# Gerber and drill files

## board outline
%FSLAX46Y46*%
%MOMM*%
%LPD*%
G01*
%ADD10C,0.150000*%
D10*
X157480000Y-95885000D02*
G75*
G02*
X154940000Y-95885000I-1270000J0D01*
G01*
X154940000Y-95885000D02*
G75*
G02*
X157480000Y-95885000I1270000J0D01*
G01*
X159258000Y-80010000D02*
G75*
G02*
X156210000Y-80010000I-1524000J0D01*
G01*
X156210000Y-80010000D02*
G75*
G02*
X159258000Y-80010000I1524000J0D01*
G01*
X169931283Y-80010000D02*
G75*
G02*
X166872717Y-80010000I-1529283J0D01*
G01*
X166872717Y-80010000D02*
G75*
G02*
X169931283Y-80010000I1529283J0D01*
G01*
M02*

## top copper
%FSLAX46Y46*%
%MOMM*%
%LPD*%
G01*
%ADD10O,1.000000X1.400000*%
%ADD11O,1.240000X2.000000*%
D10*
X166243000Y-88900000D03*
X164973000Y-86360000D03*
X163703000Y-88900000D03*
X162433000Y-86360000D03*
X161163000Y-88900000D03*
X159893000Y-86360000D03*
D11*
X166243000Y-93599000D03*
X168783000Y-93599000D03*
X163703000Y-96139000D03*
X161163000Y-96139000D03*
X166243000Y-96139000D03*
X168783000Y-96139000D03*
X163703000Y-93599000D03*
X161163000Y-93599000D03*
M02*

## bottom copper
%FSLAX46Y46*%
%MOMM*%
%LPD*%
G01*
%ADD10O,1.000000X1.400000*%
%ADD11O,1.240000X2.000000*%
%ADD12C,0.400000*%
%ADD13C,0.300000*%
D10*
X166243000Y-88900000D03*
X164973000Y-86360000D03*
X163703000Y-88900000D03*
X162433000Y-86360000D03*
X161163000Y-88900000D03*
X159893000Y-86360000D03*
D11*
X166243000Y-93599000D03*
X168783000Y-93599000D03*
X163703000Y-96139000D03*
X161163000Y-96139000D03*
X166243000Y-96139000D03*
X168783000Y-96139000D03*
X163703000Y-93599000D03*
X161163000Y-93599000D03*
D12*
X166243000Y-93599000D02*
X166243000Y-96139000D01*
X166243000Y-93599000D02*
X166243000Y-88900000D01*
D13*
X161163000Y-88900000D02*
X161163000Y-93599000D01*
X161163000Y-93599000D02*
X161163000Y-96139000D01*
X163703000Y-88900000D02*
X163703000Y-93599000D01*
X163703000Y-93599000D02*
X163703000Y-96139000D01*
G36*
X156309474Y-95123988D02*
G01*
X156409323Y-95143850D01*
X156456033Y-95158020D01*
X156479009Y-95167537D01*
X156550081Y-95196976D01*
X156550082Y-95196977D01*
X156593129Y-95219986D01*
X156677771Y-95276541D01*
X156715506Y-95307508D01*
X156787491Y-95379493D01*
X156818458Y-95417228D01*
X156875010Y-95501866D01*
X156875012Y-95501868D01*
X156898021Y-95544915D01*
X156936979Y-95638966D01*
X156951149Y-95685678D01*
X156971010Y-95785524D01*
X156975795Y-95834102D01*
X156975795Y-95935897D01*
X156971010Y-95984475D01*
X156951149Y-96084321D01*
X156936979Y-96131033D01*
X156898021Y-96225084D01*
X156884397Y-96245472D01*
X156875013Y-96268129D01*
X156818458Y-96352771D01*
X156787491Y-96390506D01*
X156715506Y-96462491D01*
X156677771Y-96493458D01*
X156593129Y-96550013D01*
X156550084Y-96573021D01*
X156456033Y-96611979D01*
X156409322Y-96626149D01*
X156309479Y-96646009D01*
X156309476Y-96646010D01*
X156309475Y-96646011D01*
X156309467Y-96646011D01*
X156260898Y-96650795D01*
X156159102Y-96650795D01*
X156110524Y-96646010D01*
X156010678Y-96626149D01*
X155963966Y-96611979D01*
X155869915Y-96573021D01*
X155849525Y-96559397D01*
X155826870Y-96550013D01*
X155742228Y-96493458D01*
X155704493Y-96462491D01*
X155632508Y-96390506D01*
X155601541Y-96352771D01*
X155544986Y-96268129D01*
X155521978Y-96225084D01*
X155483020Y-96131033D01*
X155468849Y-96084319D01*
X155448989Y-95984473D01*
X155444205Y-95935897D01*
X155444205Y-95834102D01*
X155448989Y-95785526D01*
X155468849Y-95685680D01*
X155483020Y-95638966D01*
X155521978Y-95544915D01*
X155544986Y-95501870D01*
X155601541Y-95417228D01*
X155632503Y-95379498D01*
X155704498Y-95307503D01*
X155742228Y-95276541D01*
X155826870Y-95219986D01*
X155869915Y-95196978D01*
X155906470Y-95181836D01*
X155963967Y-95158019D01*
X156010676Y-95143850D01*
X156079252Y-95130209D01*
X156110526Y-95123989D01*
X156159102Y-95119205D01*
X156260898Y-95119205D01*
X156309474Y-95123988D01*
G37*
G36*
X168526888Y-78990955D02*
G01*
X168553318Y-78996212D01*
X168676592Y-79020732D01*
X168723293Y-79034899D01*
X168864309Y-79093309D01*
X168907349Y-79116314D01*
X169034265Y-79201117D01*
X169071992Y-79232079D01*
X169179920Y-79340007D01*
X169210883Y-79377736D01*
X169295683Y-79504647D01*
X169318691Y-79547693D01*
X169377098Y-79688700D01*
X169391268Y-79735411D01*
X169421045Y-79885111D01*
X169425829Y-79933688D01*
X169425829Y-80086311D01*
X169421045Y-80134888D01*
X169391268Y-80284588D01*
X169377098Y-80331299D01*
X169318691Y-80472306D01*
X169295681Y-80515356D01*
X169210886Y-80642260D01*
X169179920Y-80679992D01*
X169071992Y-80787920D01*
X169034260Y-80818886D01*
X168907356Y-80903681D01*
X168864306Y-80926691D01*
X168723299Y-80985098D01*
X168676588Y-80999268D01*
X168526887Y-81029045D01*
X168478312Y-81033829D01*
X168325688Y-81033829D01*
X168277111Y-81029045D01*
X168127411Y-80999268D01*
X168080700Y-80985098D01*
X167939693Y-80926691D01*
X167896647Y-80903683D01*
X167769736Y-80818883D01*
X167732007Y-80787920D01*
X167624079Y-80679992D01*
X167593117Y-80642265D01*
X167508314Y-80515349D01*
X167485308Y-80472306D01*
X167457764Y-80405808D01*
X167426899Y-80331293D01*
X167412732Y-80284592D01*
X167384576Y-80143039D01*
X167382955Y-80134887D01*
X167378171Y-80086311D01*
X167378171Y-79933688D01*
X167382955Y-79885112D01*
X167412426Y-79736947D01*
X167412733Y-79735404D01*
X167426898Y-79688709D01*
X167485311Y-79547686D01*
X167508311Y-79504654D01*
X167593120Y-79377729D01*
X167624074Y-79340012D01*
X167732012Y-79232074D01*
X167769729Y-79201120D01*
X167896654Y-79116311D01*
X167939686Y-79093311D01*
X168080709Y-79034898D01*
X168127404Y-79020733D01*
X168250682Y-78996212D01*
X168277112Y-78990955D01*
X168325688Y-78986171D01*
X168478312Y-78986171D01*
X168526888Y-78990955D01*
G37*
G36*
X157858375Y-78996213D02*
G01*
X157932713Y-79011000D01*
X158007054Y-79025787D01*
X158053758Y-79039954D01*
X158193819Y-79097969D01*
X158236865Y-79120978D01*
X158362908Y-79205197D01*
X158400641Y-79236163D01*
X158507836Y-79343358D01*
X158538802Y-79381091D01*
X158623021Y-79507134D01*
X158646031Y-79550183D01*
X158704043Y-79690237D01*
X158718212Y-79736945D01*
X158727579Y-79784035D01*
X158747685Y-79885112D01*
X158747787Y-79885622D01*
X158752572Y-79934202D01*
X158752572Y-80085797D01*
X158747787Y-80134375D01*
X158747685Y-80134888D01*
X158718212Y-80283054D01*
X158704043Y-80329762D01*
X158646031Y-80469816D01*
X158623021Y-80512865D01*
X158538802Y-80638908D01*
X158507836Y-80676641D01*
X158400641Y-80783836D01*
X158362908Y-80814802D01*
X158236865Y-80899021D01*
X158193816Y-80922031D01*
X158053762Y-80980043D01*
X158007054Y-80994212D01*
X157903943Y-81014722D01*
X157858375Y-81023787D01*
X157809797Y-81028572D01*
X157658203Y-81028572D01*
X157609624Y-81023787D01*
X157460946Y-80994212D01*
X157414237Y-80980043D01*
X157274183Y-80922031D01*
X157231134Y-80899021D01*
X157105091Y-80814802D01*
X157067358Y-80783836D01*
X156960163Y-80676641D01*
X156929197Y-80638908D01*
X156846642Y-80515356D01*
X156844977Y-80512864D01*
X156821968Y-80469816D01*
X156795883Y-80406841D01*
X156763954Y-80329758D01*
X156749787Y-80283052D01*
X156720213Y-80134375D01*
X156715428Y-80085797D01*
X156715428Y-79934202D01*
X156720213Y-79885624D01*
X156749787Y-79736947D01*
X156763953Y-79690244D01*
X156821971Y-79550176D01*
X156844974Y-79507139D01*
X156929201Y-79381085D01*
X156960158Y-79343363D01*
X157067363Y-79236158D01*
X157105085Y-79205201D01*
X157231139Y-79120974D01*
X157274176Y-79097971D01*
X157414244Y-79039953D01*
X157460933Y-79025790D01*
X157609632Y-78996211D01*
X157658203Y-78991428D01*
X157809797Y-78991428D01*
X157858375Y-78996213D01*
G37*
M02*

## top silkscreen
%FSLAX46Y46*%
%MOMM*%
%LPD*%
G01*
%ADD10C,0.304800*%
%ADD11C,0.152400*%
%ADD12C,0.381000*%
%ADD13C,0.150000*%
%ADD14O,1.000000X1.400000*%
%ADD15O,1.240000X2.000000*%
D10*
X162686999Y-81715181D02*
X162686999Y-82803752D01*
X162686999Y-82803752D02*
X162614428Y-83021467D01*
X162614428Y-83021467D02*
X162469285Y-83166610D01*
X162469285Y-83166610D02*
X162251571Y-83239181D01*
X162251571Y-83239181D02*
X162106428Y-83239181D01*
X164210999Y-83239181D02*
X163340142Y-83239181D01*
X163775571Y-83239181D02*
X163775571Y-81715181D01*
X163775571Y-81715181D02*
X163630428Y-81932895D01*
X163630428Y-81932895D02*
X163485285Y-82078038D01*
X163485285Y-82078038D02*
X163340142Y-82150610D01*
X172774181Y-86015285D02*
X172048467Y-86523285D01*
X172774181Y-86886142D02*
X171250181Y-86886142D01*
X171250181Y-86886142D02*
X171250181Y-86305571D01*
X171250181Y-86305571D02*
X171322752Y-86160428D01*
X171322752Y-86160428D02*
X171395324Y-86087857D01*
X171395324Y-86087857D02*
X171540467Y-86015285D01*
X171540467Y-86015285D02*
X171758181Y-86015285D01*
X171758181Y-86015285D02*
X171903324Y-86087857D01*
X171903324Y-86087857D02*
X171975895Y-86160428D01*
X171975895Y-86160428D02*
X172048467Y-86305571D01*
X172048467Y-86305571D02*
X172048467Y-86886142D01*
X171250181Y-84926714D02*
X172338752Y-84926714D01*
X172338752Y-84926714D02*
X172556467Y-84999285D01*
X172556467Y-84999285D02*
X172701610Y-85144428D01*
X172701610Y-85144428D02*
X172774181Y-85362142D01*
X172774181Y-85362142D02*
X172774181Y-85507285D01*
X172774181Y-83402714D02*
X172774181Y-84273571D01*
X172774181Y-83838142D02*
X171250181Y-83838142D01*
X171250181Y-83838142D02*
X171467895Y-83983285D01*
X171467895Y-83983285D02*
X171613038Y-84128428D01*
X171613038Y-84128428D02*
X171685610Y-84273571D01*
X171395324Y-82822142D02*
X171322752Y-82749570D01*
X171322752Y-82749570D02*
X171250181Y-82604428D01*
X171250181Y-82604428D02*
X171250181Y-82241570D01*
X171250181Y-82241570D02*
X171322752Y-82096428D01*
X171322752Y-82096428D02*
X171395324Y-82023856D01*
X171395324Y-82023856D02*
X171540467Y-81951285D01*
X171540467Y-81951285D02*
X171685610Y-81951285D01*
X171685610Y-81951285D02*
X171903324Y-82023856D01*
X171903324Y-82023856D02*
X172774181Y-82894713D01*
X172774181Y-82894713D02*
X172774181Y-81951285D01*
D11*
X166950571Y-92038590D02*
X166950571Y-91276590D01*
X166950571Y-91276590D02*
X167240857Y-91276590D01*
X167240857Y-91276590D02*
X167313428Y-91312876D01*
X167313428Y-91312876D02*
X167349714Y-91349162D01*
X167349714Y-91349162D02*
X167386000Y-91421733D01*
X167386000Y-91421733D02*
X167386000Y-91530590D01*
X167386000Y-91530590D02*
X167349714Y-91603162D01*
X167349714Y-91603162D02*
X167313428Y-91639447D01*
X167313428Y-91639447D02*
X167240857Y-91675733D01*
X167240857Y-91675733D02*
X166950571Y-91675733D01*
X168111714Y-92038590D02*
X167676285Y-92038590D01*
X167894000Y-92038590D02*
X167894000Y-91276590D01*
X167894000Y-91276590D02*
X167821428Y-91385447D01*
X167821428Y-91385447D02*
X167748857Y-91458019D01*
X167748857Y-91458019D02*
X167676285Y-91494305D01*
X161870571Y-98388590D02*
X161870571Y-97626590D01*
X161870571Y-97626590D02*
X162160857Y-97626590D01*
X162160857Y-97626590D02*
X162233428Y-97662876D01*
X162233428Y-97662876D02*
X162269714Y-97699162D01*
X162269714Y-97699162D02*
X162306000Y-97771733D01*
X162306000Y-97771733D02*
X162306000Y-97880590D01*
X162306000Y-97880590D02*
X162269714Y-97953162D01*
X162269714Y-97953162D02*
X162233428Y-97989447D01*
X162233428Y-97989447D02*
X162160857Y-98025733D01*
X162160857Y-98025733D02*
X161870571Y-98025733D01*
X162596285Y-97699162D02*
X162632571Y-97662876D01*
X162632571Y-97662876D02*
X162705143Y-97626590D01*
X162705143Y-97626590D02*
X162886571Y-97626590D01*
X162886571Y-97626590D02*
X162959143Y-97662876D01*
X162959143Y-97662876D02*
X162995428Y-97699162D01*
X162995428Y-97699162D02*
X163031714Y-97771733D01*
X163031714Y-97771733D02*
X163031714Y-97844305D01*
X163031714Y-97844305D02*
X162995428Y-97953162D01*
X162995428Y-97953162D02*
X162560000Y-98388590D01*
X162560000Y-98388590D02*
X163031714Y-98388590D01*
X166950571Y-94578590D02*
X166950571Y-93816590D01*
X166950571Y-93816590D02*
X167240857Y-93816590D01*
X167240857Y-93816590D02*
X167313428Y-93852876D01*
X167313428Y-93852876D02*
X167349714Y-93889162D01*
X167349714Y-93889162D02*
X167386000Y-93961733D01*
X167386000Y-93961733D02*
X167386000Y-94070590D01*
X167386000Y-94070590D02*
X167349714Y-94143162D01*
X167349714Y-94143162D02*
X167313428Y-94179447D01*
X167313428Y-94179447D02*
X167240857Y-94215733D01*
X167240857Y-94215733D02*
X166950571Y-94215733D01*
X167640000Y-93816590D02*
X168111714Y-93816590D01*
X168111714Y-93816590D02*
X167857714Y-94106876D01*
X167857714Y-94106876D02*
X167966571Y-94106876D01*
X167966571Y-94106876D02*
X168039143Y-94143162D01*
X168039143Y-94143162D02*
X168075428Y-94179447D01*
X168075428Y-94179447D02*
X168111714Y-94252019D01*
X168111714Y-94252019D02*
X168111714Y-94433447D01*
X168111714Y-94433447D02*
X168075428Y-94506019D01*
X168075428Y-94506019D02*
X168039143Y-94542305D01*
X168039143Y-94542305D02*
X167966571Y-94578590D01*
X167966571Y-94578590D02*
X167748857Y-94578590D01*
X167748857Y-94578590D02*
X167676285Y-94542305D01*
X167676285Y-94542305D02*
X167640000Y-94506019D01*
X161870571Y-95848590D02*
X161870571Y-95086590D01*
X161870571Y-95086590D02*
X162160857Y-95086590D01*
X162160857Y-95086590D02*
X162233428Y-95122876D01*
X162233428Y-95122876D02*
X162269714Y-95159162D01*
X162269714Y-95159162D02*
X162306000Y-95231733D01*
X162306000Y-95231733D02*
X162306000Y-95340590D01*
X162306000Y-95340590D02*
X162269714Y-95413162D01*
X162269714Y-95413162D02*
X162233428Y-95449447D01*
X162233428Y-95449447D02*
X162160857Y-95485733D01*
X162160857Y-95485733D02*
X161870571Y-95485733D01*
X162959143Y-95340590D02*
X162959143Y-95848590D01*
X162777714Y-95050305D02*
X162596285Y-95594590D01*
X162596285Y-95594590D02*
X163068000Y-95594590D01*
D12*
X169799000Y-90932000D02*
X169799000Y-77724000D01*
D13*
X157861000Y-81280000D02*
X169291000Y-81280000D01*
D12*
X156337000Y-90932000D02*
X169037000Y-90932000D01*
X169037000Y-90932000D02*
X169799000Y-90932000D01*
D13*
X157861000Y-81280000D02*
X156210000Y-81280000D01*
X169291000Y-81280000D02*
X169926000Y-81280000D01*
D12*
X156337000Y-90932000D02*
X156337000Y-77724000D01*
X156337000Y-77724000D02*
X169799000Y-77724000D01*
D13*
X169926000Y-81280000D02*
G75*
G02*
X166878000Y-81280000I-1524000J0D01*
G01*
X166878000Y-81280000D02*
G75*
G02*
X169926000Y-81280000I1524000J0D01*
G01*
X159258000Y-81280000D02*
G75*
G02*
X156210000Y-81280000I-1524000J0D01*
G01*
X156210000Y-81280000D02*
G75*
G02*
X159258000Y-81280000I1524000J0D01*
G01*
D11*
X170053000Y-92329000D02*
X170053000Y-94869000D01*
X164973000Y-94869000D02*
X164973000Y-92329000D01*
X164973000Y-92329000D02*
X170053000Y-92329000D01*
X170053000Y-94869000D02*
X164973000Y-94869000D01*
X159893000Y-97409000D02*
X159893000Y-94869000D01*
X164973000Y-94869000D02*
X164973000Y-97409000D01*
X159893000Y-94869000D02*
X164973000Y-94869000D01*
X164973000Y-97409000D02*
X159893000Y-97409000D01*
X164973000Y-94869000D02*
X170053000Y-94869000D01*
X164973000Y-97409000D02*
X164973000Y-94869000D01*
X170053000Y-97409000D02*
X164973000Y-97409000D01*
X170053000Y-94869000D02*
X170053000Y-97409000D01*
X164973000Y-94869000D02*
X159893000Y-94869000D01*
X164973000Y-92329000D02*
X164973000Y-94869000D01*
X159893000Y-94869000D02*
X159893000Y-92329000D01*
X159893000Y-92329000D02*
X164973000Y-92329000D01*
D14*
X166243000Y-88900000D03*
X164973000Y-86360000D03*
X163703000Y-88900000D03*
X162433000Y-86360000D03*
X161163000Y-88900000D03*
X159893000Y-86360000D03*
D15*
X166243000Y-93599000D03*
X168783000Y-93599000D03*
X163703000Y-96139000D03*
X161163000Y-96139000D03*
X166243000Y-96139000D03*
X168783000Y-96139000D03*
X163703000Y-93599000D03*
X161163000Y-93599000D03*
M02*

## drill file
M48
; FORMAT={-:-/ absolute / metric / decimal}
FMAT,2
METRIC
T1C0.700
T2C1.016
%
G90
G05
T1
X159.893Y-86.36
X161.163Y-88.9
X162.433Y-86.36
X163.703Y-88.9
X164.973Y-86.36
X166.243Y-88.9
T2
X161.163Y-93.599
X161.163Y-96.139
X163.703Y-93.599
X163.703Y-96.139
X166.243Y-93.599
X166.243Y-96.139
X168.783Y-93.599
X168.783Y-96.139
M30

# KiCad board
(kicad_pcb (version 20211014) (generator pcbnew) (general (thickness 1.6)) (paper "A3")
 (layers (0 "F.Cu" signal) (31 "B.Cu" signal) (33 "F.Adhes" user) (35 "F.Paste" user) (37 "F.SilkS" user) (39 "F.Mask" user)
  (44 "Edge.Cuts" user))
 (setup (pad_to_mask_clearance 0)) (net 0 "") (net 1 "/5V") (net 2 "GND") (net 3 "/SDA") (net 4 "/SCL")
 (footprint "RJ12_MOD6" (layer "F.Cu") (at 163.195 81.28 180)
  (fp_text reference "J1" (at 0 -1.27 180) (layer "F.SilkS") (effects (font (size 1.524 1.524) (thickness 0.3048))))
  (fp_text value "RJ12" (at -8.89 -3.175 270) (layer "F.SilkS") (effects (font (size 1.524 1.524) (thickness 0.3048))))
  (fp_line (start -6.604 -9.652) (end -6.604 3.556) (layer "F.SilkS") (width 0.381))
  (fp_line (start 5.334 0) (end -6.096 0) (layer "F.SilkS") (width 0.15))
  (fp_line (start 6.858 -9.652) (end -5.842 -9.652) (layer "F.SilkS") (width 0.381))
  (fp_line (start -5.842 -9.652) (end -6.604 -9.652) (layer "F.SilkS") (width 0.381))
  (fp_line (start 5.334 0) (end 6.985 0) (layer "F.SilkS") (width 0.15))
  (fp_line (start -6.096 0) (end -6.731 0) (layer "F.SilkS") (width 0.15))
  (fp_line (start 6.858 -9.652) (end 6.858 3.556) (layer "F.SilkS") (width 0.381))
  (fp_line (start 6.858 3.556) (end -6.604 3.556) (layer "F.SilkS") (width 0.381))
  (fp_circle (center -5.207 0) (end -3.683 0) (layer "F.SilkS") (width 0.15) (fill none))
  (fp_circle (center 5.461 0) (end 6.985 0) (layer "F.SilkS") (width 0.15) (fill none))
  (pad "1" thru_hole oval locked (at -3.048 -7.62) (size 1 1.4) (drill 0.7) (layers *.Cu *.Mask "F.SilkS") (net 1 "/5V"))
  (pad "2" thru_hole oval locked (at -1.778 -5.08) (size 1 1.4) (drill 0.7) (layers *.Cu *.Mask "F.SilkS") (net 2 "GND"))
  (pad "3" thru_hole oval locked (at -0.508 -7.62) (size 1 1.4) (drill 0.7) (layers *.Cu *.Mask "F.SilkS") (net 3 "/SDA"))
  (pad "4" thru_hole oval locked (at 0.762 -5.08) (size 1 1.4) (drill 0.7) (layers *.Cu *.Mask "F.SilkS") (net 2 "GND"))
  (pad "5" thru_hole oval locked (at 2.032 -7.62) (size 1 1.4) (drill 0.7) (layers *.Cu *.Mask "F.SilkS") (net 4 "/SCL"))
  (pad "6" thru_hole oval locked (at 3.302 -5.08) (size 1 1.4) (drill 0.7) (layers *.Cu *.Mask "F.SilkS") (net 2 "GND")))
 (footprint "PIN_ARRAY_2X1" (layer "F.Cu") (at 167.513 93.599)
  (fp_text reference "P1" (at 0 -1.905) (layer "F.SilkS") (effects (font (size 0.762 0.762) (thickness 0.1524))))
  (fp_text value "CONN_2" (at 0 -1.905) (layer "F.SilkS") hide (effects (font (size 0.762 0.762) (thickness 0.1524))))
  (fp_line (start 2.54 -1.27) (end 2.54 1.27) (layer "F.SilkS") (width 0.1524))
  (fp_line (start -2.54 1.27) (end -2.54 -1.27) (layer "F.SilkS") (width 0.1524))
  (fp_line (start -2.54 -1.27) (end 2.54 -1.27) (layer "F.SilkS") (width 0.1524))
  (fp_line (start 2.54 1.27) (end -2.54 1.27) (layer "F.SilkS") (width 0.1524))
  (pad "1" thru_hole oval locked (at -1.27 0) (size 1.24 2) (drill 1.016) (layers *.Cu *.Mask "F.SilkS") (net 1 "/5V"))
  (pad "2" thru_hole oval locked (at 1.27 0) (size 1.24 2) (drill 1.016) (layers *.Cu *.Mask "F.SilkS") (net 2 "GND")))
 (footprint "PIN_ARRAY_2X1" (layer "F.Cu") (at 162.433 96.139 180)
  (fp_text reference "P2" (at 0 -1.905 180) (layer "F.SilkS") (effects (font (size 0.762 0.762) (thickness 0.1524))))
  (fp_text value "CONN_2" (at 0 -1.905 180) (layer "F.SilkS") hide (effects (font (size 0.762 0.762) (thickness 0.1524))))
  (fp_line (start 2.54 -1.27) (end 2.54 1.27) (layer "F.SilkS") (width 0.1524))
  (fp_line (start -2.54 1.27) (end -2.54 -1.27) (layer "F.SilkS") (width 0.1524))
  (fp_line (start 2.54 1.27) (end -2.54 1.27) (layer "F.SilkS") (width 0.1524))
  (fp_line (start -2.54 -1.27) (end 2.54 -1.27) (layer "F.SilkS") (width 0.1524))
  (pad "1" thru_hole oval locked (at -1.27 0 180) (size 1.24 2) (drill 1.016) (layers *.Cu *.Mask "F.SilkS") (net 3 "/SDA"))
  (pad "2" thru_hole oval locked (at 1.27 0 180) (size 1.24 2) (drill 1.016) (layers *.Cu *.Mask "F.SilkS") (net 4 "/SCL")))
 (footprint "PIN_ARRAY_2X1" (layer "F.Cu") (at 167.513 96.139)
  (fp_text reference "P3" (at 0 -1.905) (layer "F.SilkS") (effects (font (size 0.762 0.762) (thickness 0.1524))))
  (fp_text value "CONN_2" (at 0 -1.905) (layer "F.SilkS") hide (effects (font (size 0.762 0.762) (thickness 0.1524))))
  (fp_line (start -2.54 -1.27) (end 2.54 -1.27) (layer "F.SilkS") (width 0.1524))
  (fp_line (start -2.54 1.27) (end -2.54 -1.27) (layer "F.SilkS") (width 0.1524))
  (fp_line (start 2.54 1.27) (end -2.54 1.27) (layer "F.SilkS") (width 0.1524))
  (fp_line (start 2.54 -1.27) (end 2.54 1.27) (layer "F.SilkS") (width 0.1524))
  (pad "1" thru_hole oval locked (at -1.27 0) (size 1.24 2) (drill 1.016) (layers *.Cu *.Mask "F.SilkS") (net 1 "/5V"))
  (pad "2" thru_hole oval locked (at 1.27 0) (size 1.24 2) (drill 1.016) (layers *.Cu *.Mask "F.SilkS") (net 2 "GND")))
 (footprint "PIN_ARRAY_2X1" (layer "F.Cu") (at 162.433 93.599 180)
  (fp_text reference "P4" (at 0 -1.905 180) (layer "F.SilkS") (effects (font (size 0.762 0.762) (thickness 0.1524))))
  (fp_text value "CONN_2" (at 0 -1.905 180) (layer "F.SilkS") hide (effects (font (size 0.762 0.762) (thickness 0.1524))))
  (fp_line (start -2.54 -1.27) (end 2.54 -1.27) (layer "F.SilkS") (width 0.1524))
  (fp_line (start -2.54 1.27) (end -2.54 -1.27) (layer "F.SilkS") (width 0.1524))
  (fp_line (start 2.54 -1.27) (end 2.54 1.27) (layer "F.SilkS") (width 0.1524))
  (fp_line (start 2.54 1.27) (end -2.54 1.27) (layer "F.SilkS") (width 0.1524))
  (pad "1" thru_hole oval locked (at -1.27 0 180) (size 1.24 2) (drill 1.016) (layers *.Cu *.Mask "F.SilkS") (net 3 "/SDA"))
  (pad "2" thru_hole oval locked (at 1.27 0 180) (size 1.24 2) (drill 1.016) (layers *.Cu *.Mask "F.SilkS") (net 4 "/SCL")))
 (gr_circle (center 156.21 95.885) (end 157.48 95.885) (layer "Edge.Cuts") (width 0.15) (fill none))
 (gr_circle (center 157.734 80.01) (end 159.258 80.01) (layer "Edge.Cuts") (width 0.15) (fill none))
 (gr_circle (center 168.402 80.01) (end 169.926 80.137) (layer "Edge.Cuts") (width 0.15) (fill none))
 (segment (start 166.243 93.599) (end 166.243 96.139) (width 0.4) (layer "B.Cu") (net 1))
 (segment (start 166.243 93.599) (end 166.243 88.9) (width 0.4) (layer "B.Cu") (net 1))
 (segment (start 161.163 88.9) (end 161.163 93.599) (width 0.3) (layer "B.Cu") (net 4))
 (segment (start 161.163 93.599) (end 161.163 96.139) (width 0.3) (layer "B.Cu") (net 4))
 (segment (start 163.703 88.9) (end 163.703 93.599) (width 0.3) (layer "B.Cu") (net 3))
 (segment (start 163.703 93.599) (end 163.703 96.139) (width 0.3) (layer "B.Cu") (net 3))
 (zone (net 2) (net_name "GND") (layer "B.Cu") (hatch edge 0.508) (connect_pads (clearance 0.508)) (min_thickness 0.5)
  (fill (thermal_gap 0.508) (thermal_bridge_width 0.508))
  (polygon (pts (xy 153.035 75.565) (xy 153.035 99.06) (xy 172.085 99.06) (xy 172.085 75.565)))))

